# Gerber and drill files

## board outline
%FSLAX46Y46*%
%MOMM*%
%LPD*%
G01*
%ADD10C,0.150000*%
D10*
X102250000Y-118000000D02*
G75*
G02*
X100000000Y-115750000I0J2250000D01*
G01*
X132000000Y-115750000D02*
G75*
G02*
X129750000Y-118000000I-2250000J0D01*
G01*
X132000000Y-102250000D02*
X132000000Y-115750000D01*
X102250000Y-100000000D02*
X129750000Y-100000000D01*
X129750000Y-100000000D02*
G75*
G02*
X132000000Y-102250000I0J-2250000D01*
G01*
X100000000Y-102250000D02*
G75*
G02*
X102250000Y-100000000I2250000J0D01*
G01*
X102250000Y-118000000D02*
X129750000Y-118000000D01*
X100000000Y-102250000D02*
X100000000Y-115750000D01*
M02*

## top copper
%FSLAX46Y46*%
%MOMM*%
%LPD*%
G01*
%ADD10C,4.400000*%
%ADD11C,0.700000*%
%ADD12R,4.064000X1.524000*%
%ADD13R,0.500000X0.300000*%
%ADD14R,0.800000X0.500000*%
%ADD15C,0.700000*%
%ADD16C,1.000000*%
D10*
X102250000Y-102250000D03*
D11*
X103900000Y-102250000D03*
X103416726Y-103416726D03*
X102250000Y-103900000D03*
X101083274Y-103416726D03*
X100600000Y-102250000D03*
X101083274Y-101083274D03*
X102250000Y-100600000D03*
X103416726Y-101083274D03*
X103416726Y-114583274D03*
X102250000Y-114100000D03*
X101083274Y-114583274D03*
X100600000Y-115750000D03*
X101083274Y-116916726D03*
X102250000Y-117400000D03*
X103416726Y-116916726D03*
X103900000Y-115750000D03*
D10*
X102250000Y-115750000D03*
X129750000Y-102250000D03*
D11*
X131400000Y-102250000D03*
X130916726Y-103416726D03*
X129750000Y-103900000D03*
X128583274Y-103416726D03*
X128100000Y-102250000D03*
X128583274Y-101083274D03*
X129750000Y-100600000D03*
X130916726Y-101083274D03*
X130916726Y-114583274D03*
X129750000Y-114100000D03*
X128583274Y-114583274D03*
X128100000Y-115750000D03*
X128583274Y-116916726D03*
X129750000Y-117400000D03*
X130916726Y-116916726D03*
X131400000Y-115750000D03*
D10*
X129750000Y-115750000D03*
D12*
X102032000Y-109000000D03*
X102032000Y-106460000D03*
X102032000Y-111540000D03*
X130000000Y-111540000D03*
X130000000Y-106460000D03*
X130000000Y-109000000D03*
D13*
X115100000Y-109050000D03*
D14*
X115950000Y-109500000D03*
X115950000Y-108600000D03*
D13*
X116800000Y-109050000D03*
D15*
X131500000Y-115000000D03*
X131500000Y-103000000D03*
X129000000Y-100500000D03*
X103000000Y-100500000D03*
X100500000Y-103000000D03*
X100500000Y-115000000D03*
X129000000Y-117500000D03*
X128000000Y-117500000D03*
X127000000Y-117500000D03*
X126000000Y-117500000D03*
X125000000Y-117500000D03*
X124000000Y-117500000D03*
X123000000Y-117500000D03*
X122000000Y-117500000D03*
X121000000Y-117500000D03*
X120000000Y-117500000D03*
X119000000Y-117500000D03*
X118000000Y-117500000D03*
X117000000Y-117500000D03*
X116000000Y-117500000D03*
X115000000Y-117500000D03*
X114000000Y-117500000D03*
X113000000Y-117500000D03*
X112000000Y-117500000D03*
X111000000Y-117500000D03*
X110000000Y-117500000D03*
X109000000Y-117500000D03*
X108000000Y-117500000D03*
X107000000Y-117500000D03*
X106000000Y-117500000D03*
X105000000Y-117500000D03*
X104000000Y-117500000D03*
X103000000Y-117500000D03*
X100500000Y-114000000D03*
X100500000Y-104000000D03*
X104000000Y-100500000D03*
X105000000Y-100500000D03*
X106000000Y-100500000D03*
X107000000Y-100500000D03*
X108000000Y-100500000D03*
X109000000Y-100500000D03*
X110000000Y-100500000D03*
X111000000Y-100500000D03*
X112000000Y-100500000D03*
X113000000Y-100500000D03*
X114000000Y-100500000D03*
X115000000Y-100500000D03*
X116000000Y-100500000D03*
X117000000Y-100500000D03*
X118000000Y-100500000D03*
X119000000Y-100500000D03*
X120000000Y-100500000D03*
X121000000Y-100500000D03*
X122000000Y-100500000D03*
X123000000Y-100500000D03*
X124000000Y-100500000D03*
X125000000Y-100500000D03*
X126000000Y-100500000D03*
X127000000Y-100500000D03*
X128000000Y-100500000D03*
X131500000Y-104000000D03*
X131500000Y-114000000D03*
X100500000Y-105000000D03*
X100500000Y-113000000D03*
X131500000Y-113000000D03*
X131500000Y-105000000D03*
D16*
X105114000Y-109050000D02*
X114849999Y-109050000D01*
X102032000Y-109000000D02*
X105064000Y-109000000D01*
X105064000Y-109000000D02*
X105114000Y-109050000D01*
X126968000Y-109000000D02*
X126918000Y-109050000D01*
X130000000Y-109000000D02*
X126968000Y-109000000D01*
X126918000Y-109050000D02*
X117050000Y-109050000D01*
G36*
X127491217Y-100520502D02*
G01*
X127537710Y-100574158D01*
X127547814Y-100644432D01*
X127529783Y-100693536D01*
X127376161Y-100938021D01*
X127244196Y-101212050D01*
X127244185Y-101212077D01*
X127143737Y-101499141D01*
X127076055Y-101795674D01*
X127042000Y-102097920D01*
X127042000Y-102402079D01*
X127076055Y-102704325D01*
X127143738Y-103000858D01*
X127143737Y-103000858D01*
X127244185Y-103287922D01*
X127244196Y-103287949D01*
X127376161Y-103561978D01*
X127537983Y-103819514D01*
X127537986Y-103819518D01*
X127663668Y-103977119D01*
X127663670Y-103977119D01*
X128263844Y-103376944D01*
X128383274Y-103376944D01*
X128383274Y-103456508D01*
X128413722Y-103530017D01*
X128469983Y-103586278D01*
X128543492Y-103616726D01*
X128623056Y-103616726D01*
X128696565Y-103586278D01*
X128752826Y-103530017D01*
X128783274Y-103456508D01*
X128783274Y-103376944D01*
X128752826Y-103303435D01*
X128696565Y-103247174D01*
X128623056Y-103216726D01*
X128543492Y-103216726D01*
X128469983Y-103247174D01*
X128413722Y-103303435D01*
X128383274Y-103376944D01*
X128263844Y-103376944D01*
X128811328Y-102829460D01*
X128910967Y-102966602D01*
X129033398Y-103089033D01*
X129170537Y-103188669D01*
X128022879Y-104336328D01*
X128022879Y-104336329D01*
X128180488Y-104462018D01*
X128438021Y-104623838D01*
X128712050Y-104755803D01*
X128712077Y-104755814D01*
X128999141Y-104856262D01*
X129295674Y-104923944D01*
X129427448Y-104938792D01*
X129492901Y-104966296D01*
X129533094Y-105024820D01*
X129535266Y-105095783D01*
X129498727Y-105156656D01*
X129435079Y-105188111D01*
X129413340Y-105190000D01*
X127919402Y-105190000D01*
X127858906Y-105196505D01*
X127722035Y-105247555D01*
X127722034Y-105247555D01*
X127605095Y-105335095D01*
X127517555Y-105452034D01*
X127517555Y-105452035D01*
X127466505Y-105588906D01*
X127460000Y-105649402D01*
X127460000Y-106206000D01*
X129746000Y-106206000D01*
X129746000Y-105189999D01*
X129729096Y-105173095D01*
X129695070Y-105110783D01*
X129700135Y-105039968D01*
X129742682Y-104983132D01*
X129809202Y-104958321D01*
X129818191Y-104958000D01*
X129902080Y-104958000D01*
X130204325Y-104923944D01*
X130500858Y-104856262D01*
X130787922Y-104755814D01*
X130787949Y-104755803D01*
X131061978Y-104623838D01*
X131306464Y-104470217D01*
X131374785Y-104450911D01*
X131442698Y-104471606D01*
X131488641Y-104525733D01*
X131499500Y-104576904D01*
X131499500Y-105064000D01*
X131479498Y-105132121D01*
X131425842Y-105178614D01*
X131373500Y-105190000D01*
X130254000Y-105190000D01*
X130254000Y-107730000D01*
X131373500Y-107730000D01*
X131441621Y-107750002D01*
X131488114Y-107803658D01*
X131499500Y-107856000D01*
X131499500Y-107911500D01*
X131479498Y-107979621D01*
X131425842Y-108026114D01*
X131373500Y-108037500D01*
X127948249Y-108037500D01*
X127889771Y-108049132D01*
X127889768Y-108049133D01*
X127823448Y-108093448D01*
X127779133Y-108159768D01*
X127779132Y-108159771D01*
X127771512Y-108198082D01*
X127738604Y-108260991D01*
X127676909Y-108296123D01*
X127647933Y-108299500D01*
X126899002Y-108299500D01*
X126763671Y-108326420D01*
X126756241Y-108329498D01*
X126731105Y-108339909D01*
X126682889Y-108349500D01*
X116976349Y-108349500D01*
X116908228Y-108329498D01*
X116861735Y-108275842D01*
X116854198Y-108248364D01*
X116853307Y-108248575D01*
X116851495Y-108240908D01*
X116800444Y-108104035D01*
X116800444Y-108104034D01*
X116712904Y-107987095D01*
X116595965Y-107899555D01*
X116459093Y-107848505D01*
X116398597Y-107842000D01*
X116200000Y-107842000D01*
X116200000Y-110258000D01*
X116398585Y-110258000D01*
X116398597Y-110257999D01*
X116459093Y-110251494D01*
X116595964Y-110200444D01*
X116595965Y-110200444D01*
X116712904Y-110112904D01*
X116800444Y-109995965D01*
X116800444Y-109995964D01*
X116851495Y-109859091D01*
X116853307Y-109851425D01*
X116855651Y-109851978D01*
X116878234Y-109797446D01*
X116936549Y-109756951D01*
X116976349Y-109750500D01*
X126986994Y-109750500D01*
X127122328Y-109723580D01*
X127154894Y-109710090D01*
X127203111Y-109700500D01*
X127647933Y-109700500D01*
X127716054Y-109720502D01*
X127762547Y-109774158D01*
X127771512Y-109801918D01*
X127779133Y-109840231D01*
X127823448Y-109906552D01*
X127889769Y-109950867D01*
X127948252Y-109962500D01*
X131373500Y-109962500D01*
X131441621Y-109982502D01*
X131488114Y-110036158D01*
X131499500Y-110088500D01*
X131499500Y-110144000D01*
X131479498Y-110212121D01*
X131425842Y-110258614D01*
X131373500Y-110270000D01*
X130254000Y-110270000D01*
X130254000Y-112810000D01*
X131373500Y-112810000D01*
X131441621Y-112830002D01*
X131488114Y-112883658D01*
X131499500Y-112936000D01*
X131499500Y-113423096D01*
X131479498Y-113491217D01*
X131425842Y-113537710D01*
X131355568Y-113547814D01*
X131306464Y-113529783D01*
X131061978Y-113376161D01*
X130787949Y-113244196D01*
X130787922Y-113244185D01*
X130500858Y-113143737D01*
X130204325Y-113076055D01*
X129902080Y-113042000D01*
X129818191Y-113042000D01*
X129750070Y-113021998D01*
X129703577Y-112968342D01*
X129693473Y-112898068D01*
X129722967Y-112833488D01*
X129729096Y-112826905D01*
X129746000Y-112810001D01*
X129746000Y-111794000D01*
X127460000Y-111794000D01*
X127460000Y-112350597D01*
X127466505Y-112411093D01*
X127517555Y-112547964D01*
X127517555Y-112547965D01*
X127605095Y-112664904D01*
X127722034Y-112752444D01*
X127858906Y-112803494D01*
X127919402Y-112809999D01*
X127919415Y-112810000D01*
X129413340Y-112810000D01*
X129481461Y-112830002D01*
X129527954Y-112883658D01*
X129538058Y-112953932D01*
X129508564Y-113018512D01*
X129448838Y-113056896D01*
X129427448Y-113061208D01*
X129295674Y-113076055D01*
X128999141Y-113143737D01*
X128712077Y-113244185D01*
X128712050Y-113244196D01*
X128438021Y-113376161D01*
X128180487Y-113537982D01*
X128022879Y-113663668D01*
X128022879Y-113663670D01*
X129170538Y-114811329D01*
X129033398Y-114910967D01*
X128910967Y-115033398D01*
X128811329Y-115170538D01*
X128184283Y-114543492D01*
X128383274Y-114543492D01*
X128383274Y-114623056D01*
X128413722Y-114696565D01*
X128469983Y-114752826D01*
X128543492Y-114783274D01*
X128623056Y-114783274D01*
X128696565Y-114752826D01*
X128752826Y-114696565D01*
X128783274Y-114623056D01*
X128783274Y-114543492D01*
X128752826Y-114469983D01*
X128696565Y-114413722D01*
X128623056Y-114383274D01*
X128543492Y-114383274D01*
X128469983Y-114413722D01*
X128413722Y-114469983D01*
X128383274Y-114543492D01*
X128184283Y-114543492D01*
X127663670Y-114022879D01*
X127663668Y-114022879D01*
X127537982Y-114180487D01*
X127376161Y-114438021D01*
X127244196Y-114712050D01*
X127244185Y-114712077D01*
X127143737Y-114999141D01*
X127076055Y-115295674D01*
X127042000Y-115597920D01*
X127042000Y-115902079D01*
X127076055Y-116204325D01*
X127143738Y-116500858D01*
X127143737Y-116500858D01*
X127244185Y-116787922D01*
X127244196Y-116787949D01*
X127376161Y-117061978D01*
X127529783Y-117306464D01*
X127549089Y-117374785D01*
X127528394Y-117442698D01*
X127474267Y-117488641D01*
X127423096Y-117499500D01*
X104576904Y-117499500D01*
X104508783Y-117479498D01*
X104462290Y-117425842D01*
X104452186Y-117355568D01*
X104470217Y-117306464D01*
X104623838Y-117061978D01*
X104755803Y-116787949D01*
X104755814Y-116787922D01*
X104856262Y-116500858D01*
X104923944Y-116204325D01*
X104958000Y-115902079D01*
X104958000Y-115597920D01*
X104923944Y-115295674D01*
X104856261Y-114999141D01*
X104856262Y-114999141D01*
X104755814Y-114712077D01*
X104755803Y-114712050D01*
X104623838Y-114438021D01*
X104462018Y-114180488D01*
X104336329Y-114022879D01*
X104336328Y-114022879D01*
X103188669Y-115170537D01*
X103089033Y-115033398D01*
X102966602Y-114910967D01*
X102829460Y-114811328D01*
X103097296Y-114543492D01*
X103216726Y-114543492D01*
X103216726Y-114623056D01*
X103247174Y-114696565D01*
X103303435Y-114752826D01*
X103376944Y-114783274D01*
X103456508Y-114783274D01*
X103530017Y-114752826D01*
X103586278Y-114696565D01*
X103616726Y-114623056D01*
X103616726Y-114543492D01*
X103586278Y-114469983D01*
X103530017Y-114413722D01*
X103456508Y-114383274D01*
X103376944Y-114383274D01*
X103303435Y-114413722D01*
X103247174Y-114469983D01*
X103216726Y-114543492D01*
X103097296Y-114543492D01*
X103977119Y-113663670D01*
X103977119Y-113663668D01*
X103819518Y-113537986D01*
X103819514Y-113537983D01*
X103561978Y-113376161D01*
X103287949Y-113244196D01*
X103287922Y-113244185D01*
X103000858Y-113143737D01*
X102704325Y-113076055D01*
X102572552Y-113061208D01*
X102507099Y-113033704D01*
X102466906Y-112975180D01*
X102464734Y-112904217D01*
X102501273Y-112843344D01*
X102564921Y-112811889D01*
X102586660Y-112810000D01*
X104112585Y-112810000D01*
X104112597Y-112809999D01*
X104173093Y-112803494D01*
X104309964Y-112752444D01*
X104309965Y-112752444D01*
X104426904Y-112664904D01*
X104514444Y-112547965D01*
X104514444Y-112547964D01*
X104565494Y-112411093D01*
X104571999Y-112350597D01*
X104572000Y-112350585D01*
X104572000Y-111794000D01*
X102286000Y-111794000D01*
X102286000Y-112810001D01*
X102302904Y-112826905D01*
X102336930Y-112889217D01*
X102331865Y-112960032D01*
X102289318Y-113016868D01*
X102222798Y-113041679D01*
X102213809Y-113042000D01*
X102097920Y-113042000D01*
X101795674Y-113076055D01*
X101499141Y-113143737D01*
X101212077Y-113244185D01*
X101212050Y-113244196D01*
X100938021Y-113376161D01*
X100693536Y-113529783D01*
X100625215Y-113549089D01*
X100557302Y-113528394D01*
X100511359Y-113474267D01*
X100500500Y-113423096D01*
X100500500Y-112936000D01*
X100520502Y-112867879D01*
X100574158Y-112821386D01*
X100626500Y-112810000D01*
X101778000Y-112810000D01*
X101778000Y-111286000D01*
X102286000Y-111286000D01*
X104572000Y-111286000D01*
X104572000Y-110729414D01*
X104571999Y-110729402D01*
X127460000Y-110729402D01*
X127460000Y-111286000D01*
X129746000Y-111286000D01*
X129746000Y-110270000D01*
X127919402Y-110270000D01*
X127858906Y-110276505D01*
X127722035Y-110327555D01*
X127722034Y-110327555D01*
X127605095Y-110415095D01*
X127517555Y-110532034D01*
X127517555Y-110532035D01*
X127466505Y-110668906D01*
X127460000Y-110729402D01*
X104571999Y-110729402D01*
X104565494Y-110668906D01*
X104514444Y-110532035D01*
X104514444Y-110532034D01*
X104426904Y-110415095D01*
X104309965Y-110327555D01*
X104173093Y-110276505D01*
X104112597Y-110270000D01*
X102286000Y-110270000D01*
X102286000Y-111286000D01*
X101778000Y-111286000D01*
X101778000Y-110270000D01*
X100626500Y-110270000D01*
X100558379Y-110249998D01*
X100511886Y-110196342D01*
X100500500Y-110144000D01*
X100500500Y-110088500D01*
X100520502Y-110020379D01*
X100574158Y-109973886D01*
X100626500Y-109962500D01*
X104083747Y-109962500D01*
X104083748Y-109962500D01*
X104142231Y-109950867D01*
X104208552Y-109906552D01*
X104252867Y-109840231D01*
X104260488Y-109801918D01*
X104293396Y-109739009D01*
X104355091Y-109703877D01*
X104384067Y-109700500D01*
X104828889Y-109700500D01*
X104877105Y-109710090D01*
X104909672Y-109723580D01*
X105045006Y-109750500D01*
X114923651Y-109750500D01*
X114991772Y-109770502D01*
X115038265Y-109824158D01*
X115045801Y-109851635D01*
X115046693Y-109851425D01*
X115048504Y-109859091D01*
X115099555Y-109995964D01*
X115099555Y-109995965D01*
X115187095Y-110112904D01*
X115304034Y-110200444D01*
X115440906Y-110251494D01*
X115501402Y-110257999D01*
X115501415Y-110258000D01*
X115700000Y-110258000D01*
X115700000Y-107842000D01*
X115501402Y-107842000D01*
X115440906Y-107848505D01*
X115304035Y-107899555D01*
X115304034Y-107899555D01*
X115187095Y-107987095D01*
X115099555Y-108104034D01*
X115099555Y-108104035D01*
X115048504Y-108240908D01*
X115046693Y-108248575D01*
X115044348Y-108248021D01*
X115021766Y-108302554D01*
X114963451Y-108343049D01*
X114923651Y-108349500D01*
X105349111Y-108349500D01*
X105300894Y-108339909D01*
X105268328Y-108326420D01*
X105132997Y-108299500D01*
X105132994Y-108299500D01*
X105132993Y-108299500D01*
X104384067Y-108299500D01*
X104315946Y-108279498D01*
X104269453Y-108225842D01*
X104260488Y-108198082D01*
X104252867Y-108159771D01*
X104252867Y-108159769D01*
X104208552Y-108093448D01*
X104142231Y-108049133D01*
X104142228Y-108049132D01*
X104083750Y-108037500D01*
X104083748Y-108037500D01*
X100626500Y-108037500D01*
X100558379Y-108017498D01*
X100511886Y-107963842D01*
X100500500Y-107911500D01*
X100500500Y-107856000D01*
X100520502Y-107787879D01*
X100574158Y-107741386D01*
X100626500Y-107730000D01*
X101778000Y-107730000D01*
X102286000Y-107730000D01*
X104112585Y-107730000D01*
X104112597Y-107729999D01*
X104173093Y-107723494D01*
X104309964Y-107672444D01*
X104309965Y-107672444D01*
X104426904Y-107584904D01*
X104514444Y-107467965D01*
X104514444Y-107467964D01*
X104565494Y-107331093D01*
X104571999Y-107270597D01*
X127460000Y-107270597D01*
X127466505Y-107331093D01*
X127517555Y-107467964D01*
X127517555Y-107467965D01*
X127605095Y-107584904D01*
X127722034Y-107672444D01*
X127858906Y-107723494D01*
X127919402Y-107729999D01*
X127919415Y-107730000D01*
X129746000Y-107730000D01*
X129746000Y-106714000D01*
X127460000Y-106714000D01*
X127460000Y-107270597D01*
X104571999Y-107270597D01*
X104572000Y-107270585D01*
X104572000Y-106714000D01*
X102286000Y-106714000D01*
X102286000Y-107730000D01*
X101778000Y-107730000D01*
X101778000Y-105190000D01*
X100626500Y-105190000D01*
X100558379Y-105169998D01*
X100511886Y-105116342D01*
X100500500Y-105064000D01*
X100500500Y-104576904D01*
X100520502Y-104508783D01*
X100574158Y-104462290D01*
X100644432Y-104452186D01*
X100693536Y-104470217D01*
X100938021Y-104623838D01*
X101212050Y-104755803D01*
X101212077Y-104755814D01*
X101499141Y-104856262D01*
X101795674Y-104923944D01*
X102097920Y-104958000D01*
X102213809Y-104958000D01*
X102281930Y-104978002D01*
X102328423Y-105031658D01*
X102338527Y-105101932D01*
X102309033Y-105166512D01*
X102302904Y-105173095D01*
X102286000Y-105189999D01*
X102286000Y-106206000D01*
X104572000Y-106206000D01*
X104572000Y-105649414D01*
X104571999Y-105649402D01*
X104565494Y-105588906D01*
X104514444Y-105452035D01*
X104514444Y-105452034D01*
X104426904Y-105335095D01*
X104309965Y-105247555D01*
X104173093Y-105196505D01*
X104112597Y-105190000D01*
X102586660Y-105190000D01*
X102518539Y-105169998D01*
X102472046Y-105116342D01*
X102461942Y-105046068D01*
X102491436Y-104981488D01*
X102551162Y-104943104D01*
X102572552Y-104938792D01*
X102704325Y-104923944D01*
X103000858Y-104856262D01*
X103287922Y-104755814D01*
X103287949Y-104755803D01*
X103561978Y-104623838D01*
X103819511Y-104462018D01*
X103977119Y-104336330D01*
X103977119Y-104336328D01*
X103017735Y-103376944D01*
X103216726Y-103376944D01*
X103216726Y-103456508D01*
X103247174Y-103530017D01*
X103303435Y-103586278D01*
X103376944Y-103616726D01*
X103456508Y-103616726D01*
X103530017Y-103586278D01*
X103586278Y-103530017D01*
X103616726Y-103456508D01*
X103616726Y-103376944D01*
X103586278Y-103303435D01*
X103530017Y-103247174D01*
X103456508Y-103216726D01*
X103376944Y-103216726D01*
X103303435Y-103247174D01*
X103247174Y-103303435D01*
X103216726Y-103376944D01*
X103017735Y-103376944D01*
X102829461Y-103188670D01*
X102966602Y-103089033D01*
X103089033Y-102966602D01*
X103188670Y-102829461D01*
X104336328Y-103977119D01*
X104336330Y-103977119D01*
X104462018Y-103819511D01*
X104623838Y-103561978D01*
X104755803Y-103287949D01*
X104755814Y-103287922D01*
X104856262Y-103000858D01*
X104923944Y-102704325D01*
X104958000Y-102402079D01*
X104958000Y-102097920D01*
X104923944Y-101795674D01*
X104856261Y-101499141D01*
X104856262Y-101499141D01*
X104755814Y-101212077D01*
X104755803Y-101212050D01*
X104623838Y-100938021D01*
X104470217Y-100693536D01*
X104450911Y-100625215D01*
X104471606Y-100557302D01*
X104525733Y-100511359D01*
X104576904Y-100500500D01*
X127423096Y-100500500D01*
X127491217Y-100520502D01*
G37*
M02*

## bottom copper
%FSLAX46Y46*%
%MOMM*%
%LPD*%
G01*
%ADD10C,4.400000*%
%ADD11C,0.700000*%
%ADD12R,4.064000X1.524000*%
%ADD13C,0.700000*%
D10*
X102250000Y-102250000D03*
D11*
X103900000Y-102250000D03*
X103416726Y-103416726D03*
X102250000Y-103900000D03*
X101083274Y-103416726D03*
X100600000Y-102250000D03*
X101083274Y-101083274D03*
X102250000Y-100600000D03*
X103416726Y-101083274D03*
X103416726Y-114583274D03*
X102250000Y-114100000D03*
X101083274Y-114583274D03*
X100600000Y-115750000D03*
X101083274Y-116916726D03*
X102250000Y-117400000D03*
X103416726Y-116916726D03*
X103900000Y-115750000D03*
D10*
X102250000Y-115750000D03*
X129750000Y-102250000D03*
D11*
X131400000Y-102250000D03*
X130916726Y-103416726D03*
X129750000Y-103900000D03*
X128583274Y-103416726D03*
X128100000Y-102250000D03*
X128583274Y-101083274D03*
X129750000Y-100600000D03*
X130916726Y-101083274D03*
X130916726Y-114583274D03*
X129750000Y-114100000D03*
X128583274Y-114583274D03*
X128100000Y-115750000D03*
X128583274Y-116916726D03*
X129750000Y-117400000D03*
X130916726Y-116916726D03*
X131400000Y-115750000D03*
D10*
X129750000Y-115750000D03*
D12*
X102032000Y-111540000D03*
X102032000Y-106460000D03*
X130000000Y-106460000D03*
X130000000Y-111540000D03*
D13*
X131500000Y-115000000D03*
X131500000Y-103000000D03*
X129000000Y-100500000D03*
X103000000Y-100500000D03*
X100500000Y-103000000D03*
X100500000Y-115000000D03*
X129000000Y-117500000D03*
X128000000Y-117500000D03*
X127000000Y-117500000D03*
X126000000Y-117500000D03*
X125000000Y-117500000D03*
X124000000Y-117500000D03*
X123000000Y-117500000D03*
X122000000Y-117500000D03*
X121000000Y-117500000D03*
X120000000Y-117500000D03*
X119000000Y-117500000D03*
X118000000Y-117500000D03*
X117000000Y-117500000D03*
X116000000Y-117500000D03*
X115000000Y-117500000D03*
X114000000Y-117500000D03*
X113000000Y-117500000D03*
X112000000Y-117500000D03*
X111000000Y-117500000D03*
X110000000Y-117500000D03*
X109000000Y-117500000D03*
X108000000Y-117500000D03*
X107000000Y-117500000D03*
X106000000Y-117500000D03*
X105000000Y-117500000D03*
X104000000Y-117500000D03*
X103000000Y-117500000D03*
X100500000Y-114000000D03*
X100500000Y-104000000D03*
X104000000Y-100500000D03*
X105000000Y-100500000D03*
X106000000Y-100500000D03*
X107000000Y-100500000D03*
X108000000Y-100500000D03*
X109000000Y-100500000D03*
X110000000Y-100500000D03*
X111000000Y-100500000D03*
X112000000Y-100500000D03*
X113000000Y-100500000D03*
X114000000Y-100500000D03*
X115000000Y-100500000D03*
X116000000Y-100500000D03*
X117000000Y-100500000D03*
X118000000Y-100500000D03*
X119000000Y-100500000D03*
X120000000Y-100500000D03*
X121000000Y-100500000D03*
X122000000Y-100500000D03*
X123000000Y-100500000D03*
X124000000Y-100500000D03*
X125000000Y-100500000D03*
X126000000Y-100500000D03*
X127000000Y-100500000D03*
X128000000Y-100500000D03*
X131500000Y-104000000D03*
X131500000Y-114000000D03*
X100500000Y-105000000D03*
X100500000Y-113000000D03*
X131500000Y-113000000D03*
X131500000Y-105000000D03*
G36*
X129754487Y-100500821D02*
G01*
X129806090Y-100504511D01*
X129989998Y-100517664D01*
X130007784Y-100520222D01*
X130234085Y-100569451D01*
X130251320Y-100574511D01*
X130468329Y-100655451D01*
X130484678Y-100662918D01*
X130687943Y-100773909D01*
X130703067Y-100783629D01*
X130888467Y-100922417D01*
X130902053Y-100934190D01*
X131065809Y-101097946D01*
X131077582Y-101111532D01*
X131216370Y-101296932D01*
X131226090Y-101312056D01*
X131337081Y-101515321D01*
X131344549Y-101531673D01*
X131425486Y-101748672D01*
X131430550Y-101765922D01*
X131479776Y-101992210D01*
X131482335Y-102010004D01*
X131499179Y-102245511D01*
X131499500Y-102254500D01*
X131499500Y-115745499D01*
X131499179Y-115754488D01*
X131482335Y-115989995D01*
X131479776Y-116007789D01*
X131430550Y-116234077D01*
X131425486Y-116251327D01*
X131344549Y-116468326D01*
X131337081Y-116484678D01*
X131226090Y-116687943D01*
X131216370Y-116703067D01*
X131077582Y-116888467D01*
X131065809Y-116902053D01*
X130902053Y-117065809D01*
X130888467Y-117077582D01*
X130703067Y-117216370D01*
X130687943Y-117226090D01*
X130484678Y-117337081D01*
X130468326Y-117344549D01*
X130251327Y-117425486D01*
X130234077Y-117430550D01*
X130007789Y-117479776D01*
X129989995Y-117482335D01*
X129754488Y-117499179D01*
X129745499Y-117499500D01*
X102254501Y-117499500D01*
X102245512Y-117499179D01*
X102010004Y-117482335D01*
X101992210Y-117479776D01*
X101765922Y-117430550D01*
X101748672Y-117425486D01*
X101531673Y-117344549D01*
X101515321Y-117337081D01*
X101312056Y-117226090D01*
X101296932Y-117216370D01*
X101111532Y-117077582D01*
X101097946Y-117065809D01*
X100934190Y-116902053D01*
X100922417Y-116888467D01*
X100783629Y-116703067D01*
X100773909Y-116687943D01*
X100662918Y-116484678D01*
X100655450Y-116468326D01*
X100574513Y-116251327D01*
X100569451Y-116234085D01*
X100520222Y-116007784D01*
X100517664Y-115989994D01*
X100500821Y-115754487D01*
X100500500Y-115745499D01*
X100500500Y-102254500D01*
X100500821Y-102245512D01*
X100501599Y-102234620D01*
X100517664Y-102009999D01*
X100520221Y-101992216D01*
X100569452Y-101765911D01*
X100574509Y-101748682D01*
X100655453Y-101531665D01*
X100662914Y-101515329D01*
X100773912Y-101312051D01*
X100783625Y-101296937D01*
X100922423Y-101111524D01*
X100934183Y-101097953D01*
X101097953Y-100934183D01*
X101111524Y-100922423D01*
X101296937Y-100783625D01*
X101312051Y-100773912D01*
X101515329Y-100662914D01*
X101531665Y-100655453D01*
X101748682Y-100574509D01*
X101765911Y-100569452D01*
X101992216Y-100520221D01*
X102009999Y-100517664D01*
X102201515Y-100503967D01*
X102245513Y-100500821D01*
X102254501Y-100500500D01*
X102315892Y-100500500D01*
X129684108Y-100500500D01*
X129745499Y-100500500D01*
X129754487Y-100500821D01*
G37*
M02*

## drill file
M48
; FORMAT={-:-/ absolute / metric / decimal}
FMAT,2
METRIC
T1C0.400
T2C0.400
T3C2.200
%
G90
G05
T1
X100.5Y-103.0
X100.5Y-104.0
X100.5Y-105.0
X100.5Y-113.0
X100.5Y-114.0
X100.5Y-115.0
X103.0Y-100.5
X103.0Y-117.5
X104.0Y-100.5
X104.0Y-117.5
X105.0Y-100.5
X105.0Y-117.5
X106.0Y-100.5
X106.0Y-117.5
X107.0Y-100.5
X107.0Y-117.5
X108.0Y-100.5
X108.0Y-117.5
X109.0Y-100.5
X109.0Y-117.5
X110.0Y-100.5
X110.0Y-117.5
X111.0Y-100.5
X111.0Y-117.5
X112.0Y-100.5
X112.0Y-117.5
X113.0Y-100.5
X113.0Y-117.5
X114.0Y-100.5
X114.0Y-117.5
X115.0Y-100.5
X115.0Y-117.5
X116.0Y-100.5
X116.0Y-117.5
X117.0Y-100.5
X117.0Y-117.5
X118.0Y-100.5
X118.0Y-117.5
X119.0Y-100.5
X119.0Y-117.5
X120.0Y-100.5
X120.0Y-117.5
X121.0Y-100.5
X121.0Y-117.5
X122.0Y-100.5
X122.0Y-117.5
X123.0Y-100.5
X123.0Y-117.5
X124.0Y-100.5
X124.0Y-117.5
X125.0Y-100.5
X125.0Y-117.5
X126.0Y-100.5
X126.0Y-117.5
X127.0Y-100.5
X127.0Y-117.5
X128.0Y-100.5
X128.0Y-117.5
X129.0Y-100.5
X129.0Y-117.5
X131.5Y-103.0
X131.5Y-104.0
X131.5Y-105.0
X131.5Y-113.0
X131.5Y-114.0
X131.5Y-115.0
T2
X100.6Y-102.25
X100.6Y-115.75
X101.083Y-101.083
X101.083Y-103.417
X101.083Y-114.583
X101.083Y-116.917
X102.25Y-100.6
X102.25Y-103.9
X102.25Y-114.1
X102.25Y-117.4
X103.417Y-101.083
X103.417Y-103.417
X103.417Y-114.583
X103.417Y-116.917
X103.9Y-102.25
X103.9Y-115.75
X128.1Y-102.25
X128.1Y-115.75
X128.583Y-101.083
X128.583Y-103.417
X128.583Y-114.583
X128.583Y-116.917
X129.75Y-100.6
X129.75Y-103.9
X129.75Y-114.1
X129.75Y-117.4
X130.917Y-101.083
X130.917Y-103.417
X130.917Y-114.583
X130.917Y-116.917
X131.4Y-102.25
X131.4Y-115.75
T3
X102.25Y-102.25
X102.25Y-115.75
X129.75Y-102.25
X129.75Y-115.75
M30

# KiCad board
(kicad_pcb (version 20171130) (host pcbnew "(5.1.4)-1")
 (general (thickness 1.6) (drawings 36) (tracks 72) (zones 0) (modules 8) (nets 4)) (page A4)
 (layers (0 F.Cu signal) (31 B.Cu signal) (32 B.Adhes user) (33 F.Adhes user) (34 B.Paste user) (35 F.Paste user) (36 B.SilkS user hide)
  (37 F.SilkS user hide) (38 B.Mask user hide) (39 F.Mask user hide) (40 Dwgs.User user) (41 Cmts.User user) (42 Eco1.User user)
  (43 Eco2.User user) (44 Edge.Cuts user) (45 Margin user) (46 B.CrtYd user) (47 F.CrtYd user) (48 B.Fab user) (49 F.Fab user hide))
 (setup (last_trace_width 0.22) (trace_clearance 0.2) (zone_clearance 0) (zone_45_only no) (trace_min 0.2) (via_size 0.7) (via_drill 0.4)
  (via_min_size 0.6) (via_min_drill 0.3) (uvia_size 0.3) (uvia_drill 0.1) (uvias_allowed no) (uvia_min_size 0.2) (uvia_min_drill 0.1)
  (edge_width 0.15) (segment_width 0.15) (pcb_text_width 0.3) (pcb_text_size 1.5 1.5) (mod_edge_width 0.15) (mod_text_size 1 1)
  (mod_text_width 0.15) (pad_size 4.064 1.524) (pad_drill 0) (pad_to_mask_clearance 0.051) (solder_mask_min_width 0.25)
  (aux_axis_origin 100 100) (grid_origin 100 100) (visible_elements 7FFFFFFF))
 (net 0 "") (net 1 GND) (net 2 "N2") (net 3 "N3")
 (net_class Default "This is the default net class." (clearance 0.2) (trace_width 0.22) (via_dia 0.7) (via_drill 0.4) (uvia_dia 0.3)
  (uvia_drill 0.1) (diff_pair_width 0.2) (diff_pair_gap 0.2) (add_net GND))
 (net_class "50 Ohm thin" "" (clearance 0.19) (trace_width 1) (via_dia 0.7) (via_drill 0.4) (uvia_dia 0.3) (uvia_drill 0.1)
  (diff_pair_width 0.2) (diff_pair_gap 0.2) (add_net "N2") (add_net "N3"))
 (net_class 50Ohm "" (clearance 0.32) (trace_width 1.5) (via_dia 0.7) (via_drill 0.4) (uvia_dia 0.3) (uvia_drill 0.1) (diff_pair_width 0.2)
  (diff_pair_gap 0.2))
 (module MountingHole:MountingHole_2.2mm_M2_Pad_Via (layer F.Cu) (at 102.25 102.25)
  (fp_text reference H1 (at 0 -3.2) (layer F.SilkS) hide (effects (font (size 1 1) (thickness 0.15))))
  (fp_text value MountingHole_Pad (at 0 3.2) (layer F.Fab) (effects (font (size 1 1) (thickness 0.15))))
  (pad 1 thru_hole circle (at 0 0) (size 4.4 4.4) (drill 2.2) (layers *.Cu *.Mask) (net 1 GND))
  (pad 1 thru_hole circle (at 1.65 0) (size 0.7 0.7) (drill 0.4) (layers *.Cu *.Mask) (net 1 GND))
  (pad 1 thru_hole circle (at 1.166726 1.166726) (size 0.7 0.7) (drill 0.4) (layers *.Cu *.Mask) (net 1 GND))
  (pad 1 thru_hole circle (at 0 1.65) (size 0.7 0.7) (drill 0.4) (layers *.Cu *.Mask) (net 1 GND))
  (pad 1 thru_hole circle (at -1.166726 1.166726) (size 0.7 0.7) (drill 0.4) (layers *.Cu *.Mask) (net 1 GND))
  (pad 1 thru_hole circle (at -1.65 0) (size 0.7 0.7) (drill 0.4) (layers *.Cu *.Mask) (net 1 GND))
  (pad 1 thru_hole circle (at -1.166726 -1.166726) (size 0.7 0.7) (drill 0.4) (layers *.Cu *.Mask) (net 1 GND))
  (pad 1 thru_hole circle (at 0 -1.65) (size 0.7 0.7) (drill 0.4) (layers *.Cu *.Mask) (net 1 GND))
  (pad 1 thru_hole circle (at 1.166726 -1.166726) (size 0.7 0.7) (drill 0.4) (layers *.Cu *.Mask) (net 1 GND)))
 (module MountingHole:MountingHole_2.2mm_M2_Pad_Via (layer F.Cu) (at 102.25 115.75)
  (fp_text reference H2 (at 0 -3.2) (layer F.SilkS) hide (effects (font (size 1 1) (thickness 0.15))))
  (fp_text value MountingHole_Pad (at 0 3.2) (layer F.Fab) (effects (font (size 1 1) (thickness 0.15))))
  (pad 1 thru_hole circle (at 1.166726 -1.166726) (size 0.7 0.7) (drill 0.4) (layers *.Cu *.Mask) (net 1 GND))
  (pad 1 thru_hole circle (at 0 -1.65) (size 0.7 0.7) (drill 0.4) (layers *.Cu *.Mask) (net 1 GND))
  (pad 1 thru_hole circle (at -1.166726 -1.166726) (size 0.7 0.7) (drill 0.4) (layers *.Cu *.Mask) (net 1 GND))
  (pad 1 thru_hole circle (at -1.65 0) (size 0.7 0.7) (drill 0.4) (layers *.Cu *.Mask) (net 1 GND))
  (pad 1 thru_hole circle (at -1.166726 1.166726) (size 0.7 0.7) (drill 0.4) (layers *.Cu *.Mask) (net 1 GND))
  (pad 1 thru_hole circle (at 0 1.65) (size 0.7 0.7) (drill 0.4) (layers *.Cu *.Mask) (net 1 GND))
  (pad 1 thru_hole circle (at 1.166726 1.166726) (size 0.7 0.7) (drill 0.4) (layers *.Cu *.Mask) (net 1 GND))
  (pad 1 thru_hole circle (at 1.65 0) (size 0.7 0.7) (drill 0.4) (layers *.Cu *.Mask) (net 1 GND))
  (pad 1 thru_hole circle (at 0 0) (size 4.4 4.4) (drill 2.2) (layers *.Cu *.Mask) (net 1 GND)))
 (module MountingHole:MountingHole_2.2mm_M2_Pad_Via (layer F.Cu) (at 129.75 102.25)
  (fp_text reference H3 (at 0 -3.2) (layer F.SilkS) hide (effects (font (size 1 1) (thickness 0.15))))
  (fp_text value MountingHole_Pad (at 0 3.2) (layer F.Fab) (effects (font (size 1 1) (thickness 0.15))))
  (pad 1 thru_hole circle (at 0 0) (size 4.4 4.4) (drill 2.2) (layers *.Cu *.Mask) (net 1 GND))
  (pad 1 thru_hole circle (at 1.65 0) (size 0.7 0.7) (drill 0.4) (layers *.Cu *.Mask) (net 1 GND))
  (pad 1 thru_hole circle (at 1.166726 1.166726) (size 0.7 0.7) (drill 0.4) (layers *.Cu *.Mask) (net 1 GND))
  (pad 1 thru_hole circle (at 0 1.65) (size 0.7 0.7) (drill 0.4) (layers *.Cu *.Mask) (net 1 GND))
  (pad 1 thru_hole circle (at -1.166726 1.166726) (size 0.7 0.7) (drill 0.4) (layers *.Cu *.Mask) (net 1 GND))
  (pad 1 thru_hole circle (at -1.65 0) (size 0.7 0.7) (drill 0.4) (layers *.Cu *.Mask) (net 1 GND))
  (pad 1 thru_hole circle (at -1.166726 -1.166726) (size 0.7 0.7) (drill 0.4) (layers *.Cu *.Mask) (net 1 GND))
  (pad 1 thru_hole circle (at 0 -1.65) (size 0.7 0.7) (drill 0.4) (layers *.Cu *.Mask) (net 1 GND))
  (pad 1 thru_hole circle (at 1.166726 -1.166726) (size 0.7 0.7) (drill 0.4) (layers *.Cu *.Mask) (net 1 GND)))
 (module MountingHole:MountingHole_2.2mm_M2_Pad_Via (layer F.Cu) (at 129.75 115.75)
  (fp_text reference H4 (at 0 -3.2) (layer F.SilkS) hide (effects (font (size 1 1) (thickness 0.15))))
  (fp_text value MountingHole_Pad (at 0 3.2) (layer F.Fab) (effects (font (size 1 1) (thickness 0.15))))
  (pad 1 thru_hole circle (at 1.166726 -1.166726) (size 0.7 0.7) (drill 0.4) (layers *.Cu *.Mask) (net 1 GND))
  (pad 1 thru_hole circle (at 0 -1.65) (size 0.7 0.7) (drill 0.4) (layers *.Cu *.Mask) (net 1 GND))
  (pad 1 thru_hole circle (at -1.166726 -1.166726) (size 0.7 0.7) (drill 0.4) (layers *.Cu *.Mask) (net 1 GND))
  (pad 1 thru_hole circle (at -1.65 0) (size 0.7 0.7) (drill 0.4) (layers *.Cu *.Mask) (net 1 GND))
  (pad 1 thru_hole circle (at -1.166726 1.166726) (size 0.7 0.7) (drill 0.4) (layers *.Cu *.Mask) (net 1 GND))
  (pad 1 thru_hole circle (at 0 1.65) (size 0.7 0.7) (drill 0.4) (layers *.Cu *.Mask) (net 1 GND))
  (pad 1 thru_hole circle (at 1.166726 1.166726) (size 0.7 0.7) (drill 0.4) (layers *.Cu *.Mask) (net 1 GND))
  (pad 1 thru_hole circle (at 1.65 0) (size 0.7 0.7) (drill 0.4) (layers *.Cu *.Mask) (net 1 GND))
  (pad 1 thru_hole circle (at 0 0) (size 4.4 4.4) (drill 2.2) (layers *.Cu *.Mask) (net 1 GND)))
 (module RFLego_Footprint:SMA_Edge (layer F.Cu) (at 100 109)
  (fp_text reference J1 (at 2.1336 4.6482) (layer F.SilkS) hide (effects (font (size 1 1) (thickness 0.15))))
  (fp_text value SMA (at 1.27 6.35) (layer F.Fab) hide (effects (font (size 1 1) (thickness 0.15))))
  (pad 1 smd rect (at 2.032 0) (size 4.064 1.524) (layers F.Cu F.Mask) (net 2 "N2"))
  (pad 2 smd rect (at 2.032 -2.54) (size 4.064 1.524) (layers F.Cu F.Mask) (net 1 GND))
  (pad 2 smd rect (at 2.032 2.54) (size 4.064 1.524) (layers B.Cu B.Mask) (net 1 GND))
  (pad 2 smd rect (at 2.032 -2.54) (size 4.064 1.524) (layers B.Cu B.Mask) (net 1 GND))
  (pad 2 smd rect (at 2.032 2.54) (size 4.064 1.524) (layers F.Cu F.Mask) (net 1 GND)))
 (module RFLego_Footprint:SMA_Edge (layer F.Cu) (at 127.968 109)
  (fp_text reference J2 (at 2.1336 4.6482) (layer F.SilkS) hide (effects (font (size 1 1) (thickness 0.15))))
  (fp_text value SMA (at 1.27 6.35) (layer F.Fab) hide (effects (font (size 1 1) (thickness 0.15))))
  (pad 2 smd rect (at 2.032 2.54) (size 4.064 1.524) (layers F.Cu F.Mask) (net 1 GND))
  (pad 2 smd rect (at 2.032 -2.54) (size 4.064 1.524) (layers B.Cu B.Mask) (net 1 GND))
  (pad 2 smd rect (at 2.032 2.54) (size 4.064 1.524) (layers B.Cu B.Mask) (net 1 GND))
  (pad 2 smd rect (at 2.032 -2.54) (size 4.064 1.524) (layers F.Cu F.Mask) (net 1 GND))
  (pad 1 smd rect (at 2.032 0) (size 4.064 1.524) (layers F.Cu F.Mask) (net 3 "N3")))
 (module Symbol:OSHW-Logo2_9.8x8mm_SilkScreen (layer B.Cu) (at 109.5 113.25 180)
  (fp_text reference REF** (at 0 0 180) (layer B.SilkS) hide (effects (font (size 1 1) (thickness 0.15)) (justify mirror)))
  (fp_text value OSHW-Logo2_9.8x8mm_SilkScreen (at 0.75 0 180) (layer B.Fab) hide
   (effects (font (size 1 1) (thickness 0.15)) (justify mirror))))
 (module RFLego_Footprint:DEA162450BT (layer F.Cu) (at 115.1 109.05)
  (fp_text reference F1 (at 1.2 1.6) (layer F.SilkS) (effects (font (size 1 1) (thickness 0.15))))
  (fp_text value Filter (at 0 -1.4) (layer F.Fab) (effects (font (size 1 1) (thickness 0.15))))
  (pad 1 smd rect (at 0 0) (size 0.5 0.3) (layers F.Cu F.Paste F.Mask) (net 2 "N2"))
  (pad 3 smd rect (at 0.85 0.45) (size 0.8 0.5) (layers F.Cu F.Paste F.Mask) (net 1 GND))
  (pad 3 smd rect (at 0.85 -0.45) (size 0.8 0.5) (layers F.Cu F.Paste F.Mask) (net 1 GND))
  (pad 2 smd rect (at 1.7 0) (size 0.5 0.3) (layers F.Cu F.Paste F.Mask) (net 3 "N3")))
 (gr_arc (start 102.25 115.75) (end 100 115.75) (angle -90) (layer Edge.Cuts) (width 0.15))
 (gr_arc (start 129.75 115.75) (end 129.75 118) (angle -90) (layer Edge.Cuts) (width 0.15))
 (gr_line (start 132 102.25) (end 132 115.75) (layer Edge.Cuts) (width 0.15))
 (gr_line (start 102.25 100) (end 129.75 100) (layer Edge.Cuts) (width 0.15))
 (gr_arc (start 129.75 102.25) (end 132 102.25) (angle -90) (layer Edge.Cuts) (width 0.15))
 (gr_arc (start 102.25 102.25) (end 102.25 100) (angle -90) (layer Edge.Cuts) (width 0.15))
 (gr_line (start 102.25 118) (end 129.75 118) (layer Edge.Cuts) (width 0.15))
 (gr_line (start 100 102.25) (end 100 115.75) (layer Edge.Cuts) (width 0.15))
 (via (at 131.5 115) (size 0.7) (drill 0.4) (layers F.Cu B.Cu) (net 1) (status 30))
 (via (at 131.5 103) (size 0.7) (drill 0.4) (layers F.Cu B.Cu) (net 1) (status 30))
 (via (at 129 100.5) (size 0.7) (drill 0.4) (layers F.Cu B.Cu) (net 1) (status 30))
 (via (at 103 100.5) (size 0.7) (drill 0.4) (layers F.Cu B.Cu) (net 1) (status 30))
 (via (at 100.5 103) (size 0.7) (drill 0.4) (layers F.Cu B.Cu) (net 1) (status 30))
 (via (at 100.5 115) (size 0.7) (drill 0.4) (layers F.Cu B.Cu) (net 1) (status 30))
 (via (at 129 117.5) (size 0.7) (drill 0.4) (layers F.Cu B.Cu) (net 1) (status 30))
 (via (at 128 117.5) (size 0.7) (drill 0.4) (layers F.Cu B.Cu) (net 1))
 (via (at 127 117.5) (size 0.7) (drill 0.4) (layers F.Cu B.Cu) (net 1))
 (via (at 126 117.5) (size 0.7) (drill 0.4) (layers F.Cu B.Cu) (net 1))
 (via (at 125 117.5) (size 0.7) (drill 0.4) (layers F.Cu B.Cu) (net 1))
 (via (at 124 117.5) (size 0.7) (drill 0.4) (layers F.Cu B.Cu) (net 1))
 (via (at 123 117.5) (size 0.7) (drill 0.4) (layers F.Cu B.Cu) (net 1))
 (via (at 122 117.5) (size 0.7) (drill 0.4) (layers F.Cu B.Cu) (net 1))
 (via (at 121 117.5) (size 0.7) (drill 0.4) (layers F.Cu B.Cu) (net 1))
 (via (at 120 117.5) (size 0.7) (drill 0.4) (layers F.Cu B.Cu) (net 1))
 (via (at 119 117.5) (size 0.7) (drill 0.4) (layers F.Cu B.Cu) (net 1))
 (via (at 118 117.5) (size 0.7) (drill 0.4) (layers F.Cu B.Cu) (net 1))
 (via (at 117 117.5) (size 0.7) (drill 0.4) (layers F.Cu B.Cu) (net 1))
 (via (at 116 117.5) (size 0.7) (drill 0.4) (layers F.Cu B.Cu) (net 1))
 (via (at 115 117.5) (size 0.7) (drill 0.4) (layers F.Cu B.Cu) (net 1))
 (via (at 114 117.5) (size 0.7) (drill 0.4) (layers F.Cu B.Cu) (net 1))
 (via (at 113 117.5) (size 0.7) (drill 0.4) (layers F.Cu B.Cu) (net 1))
 (via (at 112 117.5) (size 0.7) (drill 0.4) (layers F.Cu B.Cu) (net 1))
 (via (at 111 117.5) (size 0.7) (drill 0.4) (layers F.Cu B.Cu) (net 1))
 (via (at 110 117.5) (size 0.7) (drill 0.4) (layers F.Cu B.Cu) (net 1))
 (via (at 109 117.5) (size 0.7) (drill 0.4) (layers F.Cu B.Cu) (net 1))
 (via (at 108 117.5) (size 0.7) (drill 0.4) (layers F.Cu B.Cu) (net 1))
 (via (at 107 117.5) (size 0.7) (drill 0.4) (layers F.Cu B.Cu) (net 1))
 (via (at 106 117.5) (size 0.7) (drill 0.4) (layers F.Cu B.Cu) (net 1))
 (via (at 105 117.5) (size 0.7) (drill 0.4) (layers F.Cu B.Cu) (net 1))
 (via (at 104 117.5) (size 0.7) (drill 0.4) (layers F.Cu B.Cu) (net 1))
 (via (at 103 117.5) (size 0.7) (drill 0.4) (layers F.Cu B.Cu) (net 1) (status 30))
 (via (at 100.5 114) (size 0.7) (drill 0.4) (layers F.Cu B.Cu) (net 1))
 (via (at 100.5 104) (size 0.7) (drill 0.4) (layers F.Cu B.Cu) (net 1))
 (via (at 104 100.5) (size 0.7) (drill 0.4) (layers F.Cu B.Cu) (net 1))
 (via (at 105 100.5) (size 0.7) (drill 0.4) (layers F.Cu B.Cu) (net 1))
 (via (at 106 100.5) (size 0.7) (drill 0.4) (layers F.Cu B.Cu) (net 1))
 (via (at 107 100.5) (size 0.7) (drill 0.4) (layers F.Cu B.Cu) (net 1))
 (via (at 108 100.5) (size 0.7) (drill 0.4) (layers F.Cu B.Cu) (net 1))
 (via (at 109 100.5) (size 0.7) (drill 0.4) (layers F.Cu B.Cu) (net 1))
 (via (at 110 100.5) (size 0.7) (drill 0.4) (layers F.Cu B.Cu) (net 1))
 (via (at 111 100.5) (size 0.7) (drill 0.4) (layers F.Cu B.Cu) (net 1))
 (via (at 112 100.5) (size 0.7) (drill 0.4) (layers F.Cu B.Cu) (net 1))
 (via (at 113 100.5) (size 0.7) (drill 0.4) (layers F.Cu B.Cu) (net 1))
 (via (at 114 100.5) (size 0.7) (drill 0.4) (layers F.Cu B.Cu) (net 1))
 (via (at 115 100.5) (size 0.7) (drill 0.4) (layers F.Cu B.Cu) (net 1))
 (via (at 116 100.5) (size 0.7) (drill 0.4) (layers F.Cu B.Cu) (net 1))
 (via (at 117 100.5) (size 0.7) (drill 0.4) (layers F.Cu B.Cu) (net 1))
 (via (at 118 100.5) (size 0.7) (drill 0.4) (layers F.Cu B.Cu) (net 1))
 (via (at 119 100.5) (size 0.7) (drill 0.4) (layers F.Cu B.Cu) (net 1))
 (via (at 120 100.5) (size 0.7) (drill 0.4) (layers F.Cu B.Cu) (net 1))
 (via (at 121 100.5) (size 0.7) (drill 0.4) (layers F.Cu B.Cu) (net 1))
 (via (at 122 100.5) (size 0.7) (drill 0.4) (layers F.Cu B.Cu) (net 1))
 (via (at 123 100.5) (size 0.7) (drill 0.4) (layers F.Cu B.Cu) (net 1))
 (via (at 124 100.5) (size 0.7) (drill 0.4) (layers F.Cu B.Cu) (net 1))
 (via (at 125 100.5) (size 0.7) (drill 0.4) (layers F.Cu B.Cu) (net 1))
 (via (at 126 100.5) (size 0.7) (drill 0.4) (layers F.Cu B.Cu) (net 1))
 (via (at 127 100.5) (size 0.7) (drill 0.4) (layers F.Cu B.Cu) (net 1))
 (via (at 128 100.5) (size 0.7) (drill 0.4) (layers F.Cu B.Cu) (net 1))
 (via (at 131.5 104) (size 0.7) (drill 0.4) (layers F.Cu B.Cu) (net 1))
 (via (at 131.5 114) (size 0.7) (drill 0.4) (layers F.Cu B.Cu) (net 1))
 (via (at 100.5 105) (size 0.7) (drill 0.4) (layers F.Cu B.Cu) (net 1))
 (via (at 100.5 113) (size 0.7) (drill 0.4) (layers F.Cu B.Cu) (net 1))
 (via (at 131.5 113) (size 0.7) (drill 0.4) (layers F.Cu B.Cu) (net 1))
 (via (at 131.5 105) (size 0.7) (drill 0.4) (layers F.Cu B.Cu) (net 1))
 (segment (start 105.114 109.05) (end 114.849999 109.05) (width 1) (layer F.Cu) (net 2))
 (segment (start 102.032 109) (end 105.064 109) (width 1) (layer F.Cu) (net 2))
 (segment (start 105.064 109) (end 105.114 109.05) (width 1) (layer F.Cu) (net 2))
 (segment (start 126.968 109) (end 126.918 109.05) (width 1) (layer F.Cu) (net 3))
 (segment (start 130 109) (end 126.968 109) (width 1) (layer F.Cu) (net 3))
 (segment (start 126.918 109.05) (end 117.05 109.05) (width 1) (layer F.Cu) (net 3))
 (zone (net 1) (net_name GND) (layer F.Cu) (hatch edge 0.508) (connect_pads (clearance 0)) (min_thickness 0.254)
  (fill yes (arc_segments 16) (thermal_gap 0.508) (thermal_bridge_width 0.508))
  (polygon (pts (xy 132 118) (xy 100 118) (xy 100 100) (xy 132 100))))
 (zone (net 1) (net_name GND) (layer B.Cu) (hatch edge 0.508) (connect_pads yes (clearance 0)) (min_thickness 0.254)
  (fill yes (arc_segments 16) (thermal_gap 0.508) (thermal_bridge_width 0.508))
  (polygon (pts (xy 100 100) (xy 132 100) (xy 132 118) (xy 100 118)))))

